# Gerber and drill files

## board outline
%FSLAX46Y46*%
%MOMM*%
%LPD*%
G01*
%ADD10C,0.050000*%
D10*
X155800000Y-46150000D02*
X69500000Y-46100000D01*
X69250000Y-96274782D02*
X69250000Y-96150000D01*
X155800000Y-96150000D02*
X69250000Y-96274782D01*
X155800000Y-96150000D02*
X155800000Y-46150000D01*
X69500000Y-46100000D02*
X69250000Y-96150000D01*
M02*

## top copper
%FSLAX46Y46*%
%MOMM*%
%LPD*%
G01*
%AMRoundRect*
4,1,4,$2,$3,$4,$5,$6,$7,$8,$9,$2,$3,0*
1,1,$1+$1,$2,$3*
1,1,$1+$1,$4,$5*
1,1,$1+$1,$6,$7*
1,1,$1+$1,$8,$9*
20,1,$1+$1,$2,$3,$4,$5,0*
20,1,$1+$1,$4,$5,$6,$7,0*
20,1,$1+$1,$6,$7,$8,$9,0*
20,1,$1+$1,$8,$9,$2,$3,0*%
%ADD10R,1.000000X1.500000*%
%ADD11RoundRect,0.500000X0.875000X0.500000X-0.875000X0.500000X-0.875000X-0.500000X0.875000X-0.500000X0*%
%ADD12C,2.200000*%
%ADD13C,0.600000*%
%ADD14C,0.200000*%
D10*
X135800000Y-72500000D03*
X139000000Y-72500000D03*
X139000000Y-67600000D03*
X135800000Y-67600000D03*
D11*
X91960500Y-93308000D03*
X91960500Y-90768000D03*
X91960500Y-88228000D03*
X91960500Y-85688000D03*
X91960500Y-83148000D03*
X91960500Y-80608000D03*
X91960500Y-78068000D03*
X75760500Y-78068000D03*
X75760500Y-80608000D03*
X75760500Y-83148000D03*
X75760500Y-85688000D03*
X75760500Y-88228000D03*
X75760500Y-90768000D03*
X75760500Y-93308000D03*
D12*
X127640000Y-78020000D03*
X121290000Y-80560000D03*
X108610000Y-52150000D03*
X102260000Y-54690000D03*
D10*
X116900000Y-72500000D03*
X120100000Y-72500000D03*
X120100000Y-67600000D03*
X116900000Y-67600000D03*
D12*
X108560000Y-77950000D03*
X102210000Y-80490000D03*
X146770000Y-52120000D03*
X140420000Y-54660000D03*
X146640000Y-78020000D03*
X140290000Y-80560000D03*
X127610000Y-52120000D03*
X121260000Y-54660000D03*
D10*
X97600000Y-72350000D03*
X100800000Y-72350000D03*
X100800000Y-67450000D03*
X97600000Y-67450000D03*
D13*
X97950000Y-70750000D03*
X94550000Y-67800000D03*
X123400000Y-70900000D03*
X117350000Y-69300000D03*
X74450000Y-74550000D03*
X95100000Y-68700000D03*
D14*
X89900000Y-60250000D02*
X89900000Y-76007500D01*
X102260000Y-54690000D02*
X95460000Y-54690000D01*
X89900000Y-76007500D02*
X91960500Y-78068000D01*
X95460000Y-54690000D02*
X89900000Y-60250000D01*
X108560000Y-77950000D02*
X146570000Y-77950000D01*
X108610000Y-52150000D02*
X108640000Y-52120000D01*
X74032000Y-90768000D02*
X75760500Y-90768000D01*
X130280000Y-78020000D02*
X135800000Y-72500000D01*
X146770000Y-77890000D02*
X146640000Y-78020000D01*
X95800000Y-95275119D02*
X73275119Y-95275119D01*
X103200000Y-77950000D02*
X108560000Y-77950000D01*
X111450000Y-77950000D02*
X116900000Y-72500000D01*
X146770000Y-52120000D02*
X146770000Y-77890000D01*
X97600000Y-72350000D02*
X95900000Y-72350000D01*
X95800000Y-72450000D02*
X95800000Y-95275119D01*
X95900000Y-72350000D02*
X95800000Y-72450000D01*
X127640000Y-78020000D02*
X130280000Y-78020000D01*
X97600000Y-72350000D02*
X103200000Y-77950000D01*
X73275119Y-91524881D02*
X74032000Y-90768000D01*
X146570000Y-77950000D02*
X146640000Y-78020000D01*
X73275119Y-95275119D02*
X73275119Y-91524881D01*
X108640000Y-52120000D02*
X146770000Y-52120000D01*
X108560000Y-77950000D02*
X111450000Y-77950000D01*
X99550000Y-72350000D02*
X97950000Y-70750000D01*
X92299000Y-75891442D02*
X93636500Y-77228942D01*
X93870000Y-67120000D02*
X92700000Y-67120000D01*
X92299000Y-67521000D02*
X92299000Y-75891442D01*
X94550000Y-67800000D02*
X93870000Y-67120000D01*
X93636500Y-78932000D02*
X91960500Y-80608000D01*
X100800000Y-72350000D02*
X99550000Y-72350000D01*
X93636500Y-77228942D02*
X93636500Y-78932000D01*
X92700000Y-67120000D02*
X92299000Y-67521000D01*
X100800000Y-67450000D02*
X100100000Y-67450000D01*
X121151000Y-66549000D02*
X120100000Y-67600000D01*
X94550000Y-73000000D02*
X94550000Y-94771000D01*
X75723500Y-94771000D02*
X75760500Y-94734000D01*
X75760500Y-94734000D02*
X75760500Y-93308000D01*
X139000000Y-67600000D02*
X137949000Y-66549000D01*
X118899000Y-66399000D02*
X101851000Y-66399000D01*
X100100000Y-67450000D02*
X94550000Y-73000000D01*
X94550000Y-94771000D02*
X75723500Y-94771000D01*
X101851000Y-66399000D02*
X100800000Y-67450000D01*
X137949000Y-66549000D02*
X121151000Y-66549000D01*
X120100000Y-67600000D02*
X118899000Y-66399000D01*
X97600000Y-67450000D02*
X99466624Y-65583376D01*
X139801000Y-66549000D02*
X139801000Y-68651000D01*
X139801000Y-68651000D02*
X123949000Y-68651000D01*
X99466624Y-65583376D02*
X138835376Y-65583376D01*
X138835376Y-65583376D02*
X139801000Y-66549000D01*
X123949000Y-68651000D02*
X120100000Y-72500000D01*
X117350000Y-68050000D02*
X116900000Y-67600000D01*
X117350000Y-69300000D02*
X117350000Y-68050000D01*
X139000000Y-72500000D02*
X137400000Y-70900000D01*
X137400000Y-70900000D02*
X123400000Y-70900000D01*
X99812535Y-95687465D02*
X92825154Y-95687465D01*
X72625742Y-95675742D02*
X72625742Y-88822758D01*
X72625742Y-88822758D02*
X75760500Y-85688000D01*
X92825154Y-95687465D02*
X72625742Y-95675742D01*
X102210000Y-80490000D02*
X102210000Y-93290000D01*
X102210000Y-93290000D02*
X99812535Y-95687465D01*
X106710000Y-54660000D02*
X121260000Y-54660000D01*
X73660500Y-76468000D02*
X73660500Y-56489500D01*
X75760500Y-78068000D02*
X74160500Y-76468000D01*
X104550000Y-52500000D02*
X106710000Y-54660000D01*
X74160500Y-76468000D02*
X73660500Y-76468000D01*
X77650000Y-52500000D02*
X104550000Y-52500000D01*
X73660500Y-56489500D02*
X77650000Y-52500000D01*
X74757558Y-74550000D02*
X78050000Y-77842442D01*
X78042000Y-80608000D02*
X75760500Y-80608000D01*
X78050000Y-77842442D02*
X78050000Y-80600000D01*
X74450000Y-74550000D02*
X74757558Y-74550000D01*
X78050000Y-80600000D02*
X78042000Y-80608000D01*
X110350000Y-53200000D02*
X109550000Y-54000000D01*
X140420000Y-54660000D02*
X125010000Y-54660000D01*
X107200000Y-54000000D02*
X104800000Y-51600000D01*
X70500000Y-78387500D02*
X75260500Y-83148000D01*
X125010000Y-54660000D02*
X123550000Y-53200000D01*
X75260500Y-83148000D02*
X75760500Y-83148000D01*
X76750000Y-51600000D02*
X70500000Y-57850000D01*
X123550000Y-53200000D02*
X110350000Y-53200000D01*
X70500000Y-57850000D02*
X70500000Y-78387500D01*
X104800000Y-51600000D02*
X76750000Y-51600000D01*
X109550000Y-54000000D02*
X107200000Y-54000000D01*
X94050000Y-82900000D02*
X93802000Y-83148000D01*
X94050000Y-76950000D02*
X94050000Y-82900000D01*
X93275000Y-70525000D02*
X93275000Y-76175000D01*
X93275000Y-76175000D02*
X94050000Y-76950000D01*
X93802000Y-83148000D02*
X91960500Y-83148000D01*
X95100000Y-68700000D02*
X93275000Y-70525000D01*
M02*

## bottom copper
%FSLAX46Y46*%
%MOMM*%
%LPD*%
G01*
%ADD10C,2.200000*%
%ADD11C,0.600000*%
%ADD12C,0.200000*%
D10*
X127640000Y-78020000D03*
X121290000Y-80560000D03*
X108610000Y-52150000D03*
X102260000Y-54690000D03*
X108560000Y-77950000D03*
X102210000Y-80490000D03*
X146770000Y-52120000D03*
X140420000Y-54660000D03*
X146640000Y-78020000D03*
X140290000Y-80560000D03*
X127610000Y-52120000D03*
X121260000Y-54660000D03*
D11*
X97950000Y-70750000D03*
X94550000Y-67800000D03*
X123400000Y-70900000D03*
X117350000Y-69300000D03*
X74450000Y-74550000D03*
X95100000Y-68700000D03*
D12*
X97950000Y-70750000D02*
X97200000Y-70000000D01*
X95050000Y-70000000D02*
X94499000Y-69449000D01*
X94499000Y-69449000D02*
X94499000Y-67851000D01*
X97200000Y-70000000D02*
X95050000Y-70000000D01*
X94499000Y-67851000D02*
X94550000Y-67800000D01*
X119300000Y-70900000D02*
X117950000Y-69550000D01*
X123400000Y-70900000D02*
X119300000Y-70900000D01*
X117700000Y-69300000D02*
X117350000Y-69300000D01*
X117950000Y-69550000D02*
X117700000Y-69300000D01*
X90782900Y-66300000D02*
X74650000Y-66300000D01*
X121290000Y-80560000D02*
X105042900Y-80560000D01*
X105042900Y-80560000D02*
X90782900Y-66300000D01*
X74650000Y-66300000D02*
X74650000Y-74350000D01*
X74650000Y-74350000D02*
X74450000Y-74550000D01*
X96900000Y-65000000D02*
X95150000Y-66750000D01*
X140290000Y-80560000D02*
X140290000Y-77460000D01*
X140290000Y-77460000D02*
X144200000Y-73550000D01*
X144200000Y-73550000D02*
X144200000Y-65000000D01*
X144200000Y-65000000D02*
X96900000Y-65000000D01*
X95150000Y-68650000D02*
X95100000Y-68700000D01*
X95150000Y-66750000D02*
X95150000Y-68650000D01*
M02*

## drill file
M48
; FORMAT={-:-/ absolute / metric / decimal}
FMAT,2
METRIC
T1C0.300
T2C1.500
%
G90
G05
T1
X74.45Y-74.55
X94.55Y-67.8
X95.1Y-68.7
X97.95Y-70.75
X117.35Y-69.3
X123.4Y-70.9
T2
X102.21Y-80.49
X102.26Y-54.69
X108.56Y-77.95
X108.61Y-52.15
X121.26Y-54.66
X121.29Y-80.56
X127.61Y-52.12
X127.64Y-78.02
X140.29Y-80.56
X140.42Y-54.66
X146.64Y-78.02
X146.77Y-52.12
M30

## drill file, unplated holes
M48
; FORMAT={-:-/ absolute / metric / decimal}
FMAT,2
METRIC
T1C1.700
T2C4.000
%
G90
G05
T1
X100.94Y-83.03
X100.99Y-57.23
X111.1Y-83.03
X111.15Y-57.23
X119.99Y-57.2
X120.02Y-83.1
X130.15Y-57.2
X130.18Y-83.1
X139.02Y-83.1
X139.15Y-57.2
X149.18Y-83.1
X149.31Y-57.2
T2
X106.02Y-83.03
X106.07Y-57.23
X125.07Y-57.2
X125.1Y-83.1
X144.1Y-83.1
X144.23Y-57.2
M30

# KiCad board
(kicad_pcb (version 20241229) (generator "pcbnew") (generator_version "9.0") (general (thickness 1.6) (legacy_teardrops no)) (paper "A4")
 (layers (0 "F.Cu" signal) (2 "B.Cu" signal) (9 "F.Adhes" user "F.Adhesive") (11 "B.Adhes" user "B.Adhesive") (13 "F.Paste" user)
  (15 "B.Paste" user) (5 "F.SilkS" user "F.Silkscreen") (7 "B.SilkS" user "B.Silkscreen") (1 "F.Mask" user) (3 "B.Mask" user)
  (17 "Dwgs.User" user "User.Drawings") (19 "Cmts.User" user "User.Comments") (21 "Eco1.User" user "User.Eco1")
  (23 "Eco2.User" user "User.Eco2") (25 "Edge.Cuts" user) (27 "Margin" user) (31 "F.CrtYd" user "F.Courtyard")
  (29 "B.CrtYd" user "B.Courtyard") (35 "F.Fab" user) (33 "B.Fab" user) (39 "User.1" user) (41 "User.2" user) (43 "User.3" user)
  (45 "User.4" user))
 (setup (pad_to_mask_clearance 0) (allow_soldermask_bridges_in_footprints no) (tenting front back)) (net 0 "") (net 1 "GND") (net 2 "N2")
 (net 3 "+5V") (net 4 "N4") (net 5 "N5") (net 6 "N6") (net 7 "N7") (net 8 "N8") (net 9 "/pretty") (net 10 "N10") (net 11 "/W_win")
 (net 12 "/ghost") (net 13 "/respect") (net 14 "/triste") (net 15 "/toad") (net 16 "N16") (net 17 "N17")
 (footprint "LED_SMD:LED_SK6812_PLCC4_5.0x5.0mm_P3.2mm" (layer "F.Cu") (at 137.4 70.05 90)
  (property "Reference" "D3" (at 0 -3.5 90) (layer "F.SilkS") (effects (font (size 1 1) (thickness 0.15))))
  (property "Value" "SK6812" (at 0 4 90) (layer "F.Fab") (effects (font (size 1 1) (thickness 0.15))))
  (pad "1" smd rect (at -2.45 -1.6 270) (size 1.5 1) (layers "F.Cu" "F.Mask" "F.Paste") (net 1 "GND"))
  (pad "2" smd rect (at -2.45 1.6 270) (size 1.5 1) (layers "F.Cu" "F.Mask" "F.Paste") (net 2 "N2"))
  (pad "3" smd rect (at 2.45 1.6 270) (size 1.5 1) (layers "F.Cu" "F.Mask" "F.Paste") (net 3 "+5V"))
  (pad "4" smd rect (at 2.45 -1.6 270) (size 1.5 1) (layers "F.Cu" "F.Mask" "F.Paste") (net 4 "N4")))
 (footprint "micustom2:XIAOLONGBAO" (layer "F.Cu") (at 83.8605 85.688 180)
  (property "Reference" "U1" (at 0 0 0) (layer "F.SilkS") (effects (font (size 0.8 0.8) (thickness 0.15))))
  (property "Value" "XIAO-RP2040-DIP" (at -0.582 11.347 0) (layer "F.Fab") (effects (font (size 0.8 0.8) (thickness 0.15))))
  (pad "1" smd roundrect (at -8.1 -7.62 180) (size 2.75 2) (layers "F.Cu" "F.Mask" "F.Paste") (roundrect_rratio 0.25) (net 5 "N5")
   (solder_mask_margin 0.102))
  (pad "2" smd roundrect (at -8.1 -5.08 180) (size 2.75 2) (layers "F.Cu" "F.Mask" "F.Paste") (roundrect_rratio 0.25) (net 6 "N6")
   (solder_mask_margin 0.102))
  (pad "3" smd roundrect (at -8.1 -2.54 180) (size 2.75 2) (layers "F.Cu" "F.Mask" "F.Paste") (roundrect_rratio 0.25) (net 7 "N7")
   (solder_mask_margin 0.102))
  (pad "4" smd roundrect (at -8.1 0 180) (size 2.75 2) (layers "F.Cu" "F.Mask" "F.Paste") (roundrect_rratio 0.25) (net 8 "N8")
   (solder_mask_margin 0.102))
  (pad "5" smd roundrect (at -8.1 2.54 180) (size 2.75 2) (layers "F.Cu" "F.Mask" "F.Paste") (roundrect_rratio 0.25) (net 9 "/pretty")
   (solder_mask_margin 0.102))
  (pad "6" smd roundrect (at -8.1 5.08 180) (size 2.75 2) (layers "F.Cu" "F.Mask" "F.Paste") (roundrect_rratio 0.25) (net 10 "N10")
   (solder_mask_margin 0.102))
  (pad "7" smd roundrect (at -8.1 7.62 180) (size 2.75 2) (layers "F.Cu" "F.Mask" "F.Paste") (roundrect_rratio 0.25) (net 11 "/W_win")
   (solder_mask_margin 0.102))
  (pad "8" smd roundrect (at 8.1 7.62 180) (size 2.75 2) (layers "F.Cu" "F.Mask" "F.Paste") (roundrect_rratio 0.25) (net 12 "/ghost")
   (solder_mask_margin 0.102))
  (pad "9" smd roundrect (at 8.1 5.08 180) (size 2.75 2) (layers "F.Cu" "F.Mask" "F.Paste") (roundrect_rratio 0.25) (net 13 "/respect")
   (solder_mask_margin 0.102))
  (pad "10" smd roundrect (at 8.1 2.54 180) (size 2.75 2) (layers "F.Cu" "F.Mask" "F.Paste") (roundrect_rratio 0.25) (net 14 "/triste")
   (solder_mask_margin 0.102))
  (pad "11" smd roundrect (at 8.1 0 180) (size 2.75 2) (layers "F.Cu" "F.Mask" "F.Paste") (roundrect_rratio 0.25) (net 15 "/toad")
   (solder_mask_margin 0.102))
  (pad "12" smd roundrect (at 8.1 -2.54 180) (size 2.75 2) (layers "F.Cu" "F.Mask" "F.Paste") (roundrect_rratio 0.25) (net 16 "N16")
   (solder_mask_margin 0.102))
  (pad "13" smd roundrect (at 8.1 -5.08 180) (size 2.75 2) (layers "F.Cu" "F.Mask" "F.Paste") (roundrect_rratio 0.25) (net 1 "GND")
   (solder_mask_margin 0.102))
  (pad "14" smd roundrect (at 8.1 -7.62 180) (size 2.75 2) (layers "F.Cu" "F.Mask" "F.Paste") (roundrect_rratio 0.25) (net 3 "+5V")
   (solder_mask_margin 0.102))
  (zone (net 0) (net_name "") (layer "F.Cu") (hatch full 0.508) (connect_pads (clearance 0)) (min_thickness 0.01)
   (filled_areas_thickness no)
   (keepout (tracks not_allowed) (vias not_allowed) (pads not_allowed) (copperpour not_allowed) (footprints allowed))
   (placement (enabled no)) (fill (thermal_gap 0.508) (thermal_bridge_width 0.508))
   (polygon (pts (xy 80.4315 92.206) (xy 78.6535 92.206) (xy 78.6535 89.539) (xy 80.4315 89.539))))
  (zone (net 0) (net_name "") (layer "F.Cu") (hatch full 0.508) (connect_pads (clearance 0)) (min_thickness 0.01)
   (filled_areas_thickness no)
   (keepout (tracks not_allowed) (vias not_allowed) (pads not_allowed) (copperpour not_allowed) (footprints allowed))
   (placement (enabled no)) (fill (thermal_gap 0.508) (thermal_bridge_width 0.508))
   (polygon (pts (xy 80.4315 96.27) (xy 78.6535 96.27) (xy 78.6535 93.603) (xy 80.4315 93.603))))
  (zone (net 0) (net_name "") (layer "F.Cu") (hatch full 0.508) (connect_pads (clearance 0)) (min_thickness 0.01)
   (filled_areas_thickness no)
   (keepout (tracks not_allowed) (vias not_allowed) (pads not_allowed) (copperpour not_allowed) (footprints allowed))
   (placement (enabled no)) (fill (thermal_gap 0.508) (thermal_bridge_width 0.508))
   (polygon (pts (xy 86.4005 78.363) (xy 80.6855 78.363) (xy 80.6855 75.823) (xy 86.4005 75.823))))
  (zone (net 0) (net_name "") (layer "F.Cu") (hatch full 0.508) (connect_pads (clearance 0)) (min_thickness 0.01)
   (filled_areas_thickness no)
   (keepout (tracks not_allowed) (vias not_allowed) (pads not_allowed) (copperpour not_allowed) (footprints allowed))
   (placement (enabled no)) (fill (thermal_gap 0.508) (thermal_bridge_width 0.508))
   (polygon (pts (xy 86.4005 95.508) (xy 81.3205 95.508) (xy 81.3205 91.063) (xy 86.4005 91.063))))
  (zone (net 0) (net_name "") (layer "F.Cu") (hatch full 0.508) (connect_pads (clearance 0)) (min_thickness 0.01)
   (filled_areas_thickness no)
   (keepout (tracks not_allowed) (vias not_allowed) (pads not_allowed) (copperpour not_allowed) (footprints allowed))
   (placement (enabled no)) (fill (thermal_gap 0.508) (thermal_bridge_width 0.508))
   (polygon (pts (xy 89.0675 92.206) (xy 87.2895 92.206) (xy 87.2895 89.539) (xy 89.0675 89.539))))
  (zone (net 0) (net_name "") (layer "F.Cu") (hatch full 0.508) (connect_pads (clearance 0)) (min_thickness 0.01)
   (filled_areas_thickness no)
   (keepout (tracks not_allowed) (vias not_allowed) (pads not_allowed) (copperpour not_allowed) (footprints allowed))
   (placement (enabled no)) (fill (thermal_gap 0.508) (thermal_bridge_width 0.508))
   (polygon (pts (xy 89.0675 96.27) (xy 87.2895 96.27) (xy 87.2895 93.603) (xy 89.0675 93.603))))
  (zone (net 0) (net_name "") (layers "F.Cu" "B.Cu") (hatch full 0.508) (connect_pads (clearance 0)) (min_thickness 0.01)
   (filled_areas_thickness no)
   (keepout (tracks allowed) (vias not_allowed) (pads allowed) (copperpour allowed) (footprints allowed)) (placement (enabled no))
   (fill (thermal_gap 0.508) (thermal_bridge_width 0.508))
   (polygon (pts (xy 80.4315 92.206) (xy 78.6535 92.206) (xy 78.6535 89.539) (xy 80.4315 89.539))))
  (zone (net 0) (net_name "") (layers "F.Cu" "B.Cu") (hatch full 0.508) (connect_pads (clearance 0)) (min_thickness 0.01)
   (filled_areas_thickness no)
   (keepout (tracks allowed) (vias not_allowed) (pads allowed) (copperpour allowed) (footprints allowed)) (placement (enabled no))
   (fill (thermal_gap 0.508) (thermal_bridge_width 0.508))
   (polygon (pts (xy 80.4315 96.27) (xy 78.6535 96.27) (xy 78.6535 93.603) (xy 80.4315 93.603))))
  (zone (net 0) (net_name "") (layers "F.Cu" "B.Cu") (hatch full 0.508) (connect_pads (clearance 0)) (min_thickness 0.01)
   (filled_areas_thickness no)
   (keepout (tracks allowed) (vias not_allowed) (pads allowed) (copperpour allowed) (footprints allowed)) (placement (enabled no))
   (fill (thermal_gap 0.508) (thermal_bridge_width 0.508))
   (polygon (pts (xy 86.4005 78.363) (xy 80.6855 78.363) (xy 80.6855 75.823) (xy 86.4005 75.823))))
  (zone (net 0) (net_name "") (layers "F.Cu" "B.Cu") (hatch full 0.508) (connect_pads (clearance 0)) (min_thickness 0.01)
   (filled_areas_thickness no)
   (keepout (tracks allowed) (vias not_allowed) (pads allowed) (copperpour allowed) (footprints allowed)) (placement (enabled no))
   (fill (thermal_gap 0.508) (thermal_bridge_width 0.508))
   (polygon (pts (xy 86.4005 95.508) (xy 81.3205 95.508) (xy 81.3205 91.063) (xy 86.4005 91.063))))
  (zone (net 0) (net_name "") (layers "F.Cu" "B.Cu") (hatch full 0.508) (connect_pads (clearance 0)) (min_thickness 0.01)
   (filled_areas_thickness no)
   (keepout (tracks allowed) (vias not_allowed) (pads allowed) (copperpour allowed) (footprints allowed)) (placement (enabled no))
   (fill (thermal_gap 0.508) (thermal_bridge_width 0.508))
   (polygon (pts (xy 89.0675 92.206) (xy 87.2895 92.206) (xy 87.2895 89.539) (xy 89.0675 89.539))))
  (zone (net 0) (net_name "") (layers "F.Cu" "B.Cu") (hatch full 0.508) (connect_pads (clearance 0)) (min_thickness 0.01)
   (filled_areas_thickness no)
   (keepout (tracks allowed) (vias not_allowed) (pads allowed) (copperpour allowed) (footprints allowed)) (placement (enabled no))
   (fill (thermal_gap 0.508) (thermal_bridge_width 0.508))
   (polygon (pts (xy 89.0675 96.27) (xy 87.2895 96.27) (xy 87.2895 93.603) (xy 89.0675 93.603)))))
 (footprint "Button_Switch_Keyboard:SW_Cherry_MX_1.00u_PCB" (layer "F.Cu") (at 127.64 78.02)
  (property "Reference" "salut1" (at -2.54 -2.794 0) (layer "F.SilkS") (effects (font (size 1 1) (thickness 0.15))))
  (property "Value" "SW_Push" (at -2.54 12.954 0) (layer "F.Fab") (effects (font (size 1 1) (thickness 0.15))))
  (pad "" np_thru_hole circle (at -7.62 5.08) (size 1.7 1.7) (drill 1.7) (layers "*.Cu" "*.Mask"))
  (pad "" np_thru_hole circle (at -2.54 5.08) (size 4 4) (drill 4) (layers "*.Cu" "*.Mask"))
  (pad "" np_thru_hole circle (at 2.54 5.08) (size 1.7 1.7) (drill 1.7) (layers "*.Cu" "*.Mask"))
  (pad "1" thru_hole circle (at 0 0) (size 2.2 2.2) (drill 1.5) (layers "*.Cu" "*.Mask") (remove_unused_layers no) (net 1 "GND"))
  (pad "2" thru_hole circle (at -6.35 2.54) (size 2.2 2.2) (drill 1.5) (layers "*.Cu" "*.Mask") (remove_unused_layers no)
   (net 13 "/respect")))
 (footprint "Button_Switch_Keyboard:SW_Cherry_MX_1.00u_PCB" (layer "F.Cu") (at 108.61 52.15)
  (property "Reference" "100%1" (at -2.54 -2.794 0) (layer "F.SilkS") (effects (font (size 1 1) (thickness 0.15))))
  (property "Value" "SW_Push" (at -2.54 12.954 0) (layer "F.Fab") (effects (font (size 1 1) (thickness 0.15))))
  (pad "" np_thru_hole circle (at -7.62 5.08) (size 1.7 1.7) (drill 1.7) (layers "*.Cu" "*.Mask"))
  (pad "" np_thru_hole circle (at -2.54 5.08) (size 4 4) (drill 4) (layers "*.Cu" "*.Mask"))
  (pad "" np_thru_hole circle (at 2.54 5.08) (size 1.7 1.7) (drill 1.7) (layers "*.Cu" "*.Mask"))
  (pad "1" thru_hole circle (at 0 0) (size 2.2 2.2) (drill 1.5) (layers "*.Cu" "*.Mask") (remove_unused_layers no) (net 1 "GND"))
  (pad "2" thru_hole circle (at -6.35 2.54) (size 2.2 2.2) (drill 1.5) (layers "*.Cu" "*.Mask") (remove_unused_layers no) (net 11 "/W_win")))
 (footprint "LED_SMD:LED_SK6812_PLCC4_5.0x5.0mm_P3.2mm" (layer "F.Cu") (at 118.5 70.05 90)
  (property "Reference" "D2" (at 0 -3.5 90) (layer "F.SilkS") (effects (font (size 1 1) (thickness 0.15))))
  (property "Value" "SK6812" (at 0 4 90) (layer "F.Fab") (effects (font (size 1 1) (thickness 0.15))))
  (pad "1" smd rect (at -2.45 -1.6 270) (size 1.5 1) (layers "F.Cu" "F.Mask" "F.Paste") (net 1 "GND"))
  (pad "2" smd rect (at -2.45 1.6 270) (size 1.5 1) (layers "F.Cu" "F.Mask" "F.Paste") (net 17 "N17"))
  (pad "3" smd rect (at 2.45 1.6 270) (size 1.5 1) (layers "F.Cu" "F.Mask" "F.Paste") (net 3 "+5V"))
  (pad "4" smd rect (at 2.45 -1.6 270) (size 1.5 1) (layers "F.Cu" "F.Mask" "F.Paste") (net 2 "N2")))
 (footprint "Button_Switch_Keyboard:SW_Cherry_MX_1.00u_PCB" (layer "F.Cu") (at 108.56 77.95)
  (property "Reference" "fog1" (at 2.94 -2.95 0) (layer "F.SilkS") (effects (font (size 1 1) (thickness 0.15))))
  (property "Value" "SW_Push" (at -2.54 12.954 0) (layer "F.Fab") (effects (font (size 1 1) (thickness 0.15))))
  (pad "" np_thru_hole circle (at -7.62 5.08) (size 1.7 1.7) (drill 1.7) (layers "*.Cu" "*.Mask"))
  (pad "" np_thru_hole circle (at -2.54 5.08) (size 4 4) (drill 4) (layers "*.Cu" "*.Mask"))
  (pad "" np_thru_hole circle (at 2.54 5.08) (size 1.7 1.7) (drill 1.7) (layers "*.Cu" "*.Mask"))
  (pad "1" thru_hole circle (at 0 0) (size 2.2 2.2) (drill 1.5) (layers "*.Cu" "*.Mask") (remove_unused_layers no) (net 1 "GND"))
  (pad "2" thru_hole circle (at -6.35 2.54) (size 2.2 2.2) (drill 1.5) (layers "*.Cu" "*.Mask") (remove_unused_layers no) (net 15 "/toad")))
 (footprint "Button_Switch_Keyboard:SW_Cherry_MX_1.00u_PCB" (layer "F.Cu") (at 146.77 52.12)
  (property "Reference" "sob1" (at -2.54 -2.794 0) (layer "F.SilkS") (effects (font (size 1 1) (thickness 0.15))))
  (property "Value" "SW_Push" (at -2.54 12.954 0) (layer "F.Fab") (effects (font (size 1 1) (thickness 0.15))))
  (pad "" np_thru_hole circle (at -7.62 5.08) (size 1.7 1.7) (drill 1.7) (layers "*.Cu" "*.Mask"))
  (pad "" np_thru_hole circle (at -2.54 5.08) (size 4 4) (drill 4) (layers "*.Cu" "*.Mask"))
  (pad "" np_thru_hole circle (at 2.54 5.08) (size 1.7 1.7) (drill 1.7) (layers "*.Cu" "*.Mask"))
  (pad "1" thru_hole circle (at 0 0) (size 2.2 2.2) (drill 1.5) (layers "*.Cu" "*.Mask") (remove_unused_layers no) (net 1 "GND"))
  (pad "2" thru_hole circle (at -6.35 2.54) (size 2.2 2.2) (drill 1.5) (layers "*.Cu" "*.Mask") (remove_unused_layers no) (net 14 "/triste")))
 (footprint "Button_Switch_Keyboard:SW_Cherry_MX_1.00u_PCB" (layer "F.Cu") (at 146.64 78.02)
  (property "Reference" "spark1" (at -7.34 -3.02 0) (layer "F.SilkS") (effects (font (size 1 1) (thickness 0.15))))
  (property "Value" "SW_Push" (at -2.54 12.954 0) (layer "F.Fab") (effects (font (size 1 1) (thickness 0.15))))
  (pad "" np_thru_hole circle (at -7.62 5.08) (size 1.7 1.7) (drill 1.7) (layers "*.Cu" "*.Mask"))
  (pad "" np_thru_hole circle (at -2.54 5.08) (size 4 4) (drill 4) (layers "*.Cu" "*.Mask"))
  (pad "" np_thru_hole circle (at 2.54 5.08) (size 1.7 1.7) (drill 1.7) (layers "*.Cu" "*.Mask"))
  (pad "1" thru_hole circle (at 0 0) (size 2.2 2.2) (drill 1.5) (layers "*.Cu" "*.Mask") (remove_unused_layers no) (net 1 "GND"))
  (pad "2" thru_hole circle (at -6.35 2.54) (size 2.2 2.2) (drill 1.5) (layers "*.Cu" "*.Mask") (remove_unused_layers no) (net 9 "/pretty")))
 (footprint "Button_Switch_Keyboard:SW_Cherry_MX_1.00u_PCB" (layer "F.Cu") (at 127.61 52.12)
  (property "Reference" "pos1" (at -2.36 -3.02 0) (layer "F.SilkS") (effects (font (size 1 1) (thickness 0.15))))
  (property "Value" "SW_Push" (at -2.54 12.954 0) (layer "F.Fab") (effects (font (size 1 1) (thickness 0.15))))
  (pad "" np_thru_hole circle (at -7.62 5.08) (size 1.7 1.7) (drill 1.7) (layers "*.Cu" "*.Mask"))
  (pad "" np_thru_hole circle (at -2.54 5.08) (size 4 4) (drill 4) (layers "*.Cu" "*.Mask"))
  (pad "" np_thru_hole circle (at 2.54 5.08) (size 1.7 1.7) (drill 1.7) (layers "*.Cu" "*.Mask"))
  (pad "1" thru_hole circle (at 0 0) (size 2.2 2.2) (drill 1.5) (layers "*.Cu" "*.Mask") (remove_unused_layers no) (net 1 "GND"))
  (pad "2" thru_hole circle (at -6.35 2.54) (size 2.2 2.2) (drill 1.5) (layers "*.Cu" "*.Mask") (remove_unused_layers no) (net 12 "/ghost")))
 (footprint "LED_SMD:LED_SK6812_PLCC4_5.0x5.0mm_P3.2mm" (layer "F.Cu") (at 99.2 69.9 90)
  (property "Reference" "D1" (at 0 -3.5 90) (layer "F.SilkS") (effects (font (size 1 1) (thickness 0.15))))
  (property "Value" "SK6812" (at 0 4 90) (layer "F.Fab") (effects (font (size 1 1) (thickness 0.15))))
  (pad "1" smd rect (at -2.45 -1.6 270) (size 1.5 1) (layers "F.Cu" "F.Mask" "F.Paste") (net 1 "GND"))
  (pad "2" smd rect (at -2.45 1.6 270) (size 1.5 1) (layers "F.Cu" "F.Mask" "F.Paste") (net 10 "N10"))
  (pad "3" smd rect (at 2.45 1.6 270) (size 1.5 1) (layers "F.Cu" "F.Mask" "F.Paste") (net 3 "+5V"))
  (pad "4" smd rect (at 2.45 -1.6 270) (size 1.5 1) (layers "F.Cu" "F.Mask" "F.Paste") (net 17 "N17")))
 (gr_line (start 155.8 46.15) (end 69.5 46.1) (stroke (width 0.05) (type default)) (layer "Edge.Cuts"))
 (gr_line (start 69.25 96.274782) (end 69.25 96.15) (stroke (width 0.05) (type default)) (layer "Edge.Cuts"))
 (gr_line (start 155.8 96.15) (end 69.25 96.274782) (stroke (width 0.05) (type default)) (layer "Edge.Cuts"))
 (gr_line (start 155.8 96.15) (end 155.8 46.15) (stroke (width 0.05) (type default)) (layer "Edge.Cuts"))
 (gr_line (start 69.5 46.1) (end 69.25 96.15) (stroke (width 0.05) (type default)) (layer "Edge.Cuts"))
 (segment (start 89.9 60.25) (end 89.9 76.0075) (width 0.2) (layer "F.Cu") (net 11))
 (segment (start 102.26 54.69) (end 95.46 54.69) (width 0.2) (layer "F.Cu") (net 11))
 (segment (start 89.9 76.0075) (end 91.9605 78.068) (width 0.2) (layer "F.Cu") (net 11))
 (segment (start 95.46 54.69) (end 89.9 60.25) (width 0.2) (layer "F.Cu") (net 11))
 (segment (start 89.9 60.25) (end 89.8605 60.2895) (width 0.2) (layer "F.Cu") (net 11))
 (segment (start 108.56 77.95) (end 146.57 77.95) (width 0.2) (layer "F.Cu") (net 1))
 (segment (start 108.61 52.15) (end 108.64 52.12) (width 0.2) (layer "F.Cu") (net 1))
 (segment (start 74.032 90.768) (end 75.7605 90.768) (width 0.2) (layer "F.Cu") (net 1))
 (segment (start 130.28 78.02) (end 135.8 72.5) (width 0.2) (layer "F.Cu") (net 1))
 (segment (start 146.77 77.89) (end 146.64 78.02) (width 0.2) (layer "F.Cu") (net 1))
 (segment (start 95.8 95.275119) (end 73.275119 95.275119) (width 0.2) (layer "F.Cu") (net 1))
 (segment (start 103.2 77.95) (end 108.56 77.95) (width 0.2) (layer "F.Cu") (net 1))
 (segment (start 111.45 77.95) (end 116.9 72.5) (width 0.2) (layer "F.Cu") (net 1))
 (segment (start 146.77 52.12) (end 146.77 77.89) (width 0.2) (layer "F.Cu") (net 1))
 (segment (start 97.6 72.35) (end 95.9 72.35) (width 0.2) (layer "F.Cu") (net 1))
 (segment (start 95.8 72.45) (end 95.8 95.275119) (width 0.2) (layer "F.Cu") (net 1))
 (segment (start 95.9 72.35) (end 95.8 72.45) (width 0.2) (layer "F.Cu") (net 1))
 (segment (start 127.64 78.02) (end 130.28 78.02) (width 0.2) (layer "F.Cu") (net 1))
 (segment (start 97.6 72.35) (end 103.2 77.95) (width 0.2) (layer "F.Cu") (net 1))
 (segment (start 73.275119 91.524881) (end 74.032 90.768) (width 0.2) (layer "F.Cu") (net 1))
 (segment (start 146.57 77.95) (end 146.64 78.02) (width 0.2) (layer "F.Cu") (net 1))
 (segment (start 73.275119 95.275119) (end 73.275119 91.524881) (width 0.2) (layer "F.Cu") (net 1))
 (segment (start 108.64 52.12) (end 146.77 52.12) (width 0.2) (layer "F.Cu") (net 1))
 (segment (start 108.56 77.95) (end 111.45 77.95) (width 0.2) (layer "F.Cu") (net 1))
 (segment (start 99.55 72.35) (end 97.95 70.75) (width 0.2) (layer "F.Cu") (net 10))
 (segment (start 92.299 75.891442) (end 93.6365 77.228942) (width 0.2) (layer "F.Cu") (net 10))
 (segment (start 93.87 67.12) (end 92.7 67.12) (width 0.2) (layer "F.Cu") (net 10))
 (segment (start 92.299 67.521) (end 92.299 75.891442) (width 0.2) (layer "F.Cu") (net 10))
 (segment (start 94.55 67.8) (end 93.87 67.12) (width 0.2) (layer "F.Cu") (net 10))
 (segment (start 93.6365 78.932) (end 91.9605 80.608) (width 0.2) (layer "F.Cu") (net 10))
 (segment (start 100.8 72.35) (end 99.55 72.35) (width 0.2) (layer "F.Cu") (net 10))
 (segment (start 93.6365 77.228942) (end 93.6365 78.932) (width 0.2) (layer "F.Cu") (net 10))
 (segment (start 92.7 67.12) (end 92.299 67.521) (width 0.2) (layer "F.Cu") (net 10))
 (via (at 97.95 70.75) (size 0.6) (drill 0.3) (layers "F.Cu" "B.Cu") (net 10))
 (via (at 94.55 67.8) (size 0.6) (drill 0.3) (layers "F.Cu" "B.Cu") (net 10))
 (segment (start 97.95 70.75) (end 97.2 70) (width 0.2) (layer "B.Cu") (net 10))
 (segment (start 95.05 70) (end 94.499 69.449) (width 0.2) (layer "B.Cu") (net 10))
 (segment (start 94.499 69.449) (end 94.499 67.851) (width 0.2) (layer "B.Cu") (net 10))
 (segment (start 97.2 70) (end 95.05 70) (width 0.2) (layer "B.Cu") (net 10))
 (segment (start 94.499 67.851) (end 94.55 67.8) (width 0.2) (layer "B.Cu") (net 10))
 (segment (start 100.8 67.45) (end 100.1 67.45) (width 0.2) (layer "F.Cu") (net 3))
 (segment (start 121.151 66.549) (end 120.1 67.6) (width 0.2) (layer "F.Cu") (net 3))
 (segment (start 94.55 73) (end 94.55 94.771) (width 0.2) (layer "F.Cu") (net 3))
 (segment (start 75.7235 94.771) (end 75.7605 94.734) (width 0.2) (layer "F.Cu") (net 3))
 (segment (start 75.7605 94.734) (end 75.7605 93.308) (width 0.2) (layer "F.Cu") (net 3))
 (segment (start 139 67.6) (end 137.949 66.549) (width 0.2) (layer "F.Cu") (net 3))
 (segment (start 118.899 66.399) (end 101.851 66.399) (width 0.2) (layer "F.Cu") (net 3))
 (segment (start 100.1 67.45) (end 94.55 73) (width 0.2) (layer "F.Cu") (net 3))
 (segment (start 94.55 94.771) (end 75.7235 94.771) (width 0.2) (layer "F.Cu") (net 3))
 (segment (start 101.851 66.399) (end 100.8 67.45) (width 0.2) (layer "F.Cu") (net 3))
 (segment (start 137.949 66.549) (end 121.151 66.549) (width 0.2) (layer "F.Cu") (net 3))
 (segment (start 120.1 67.6) (end 118.899 66.399) (width 0.2) (layer "F.Cu") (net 3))
 (segment (start 97.6 67.45) (end 99.466624 65.583376) (width 0.2) (layer "F.Cu") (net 17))
 (segment (start 139.801 66.549) (end 139.801 68.651) (width 0.2) (layer "F.Cu") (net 17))
 (segment (start 139.801 68.651) (end 123.949 68.651) (width 0.2) (layer "F.Cu") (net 17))
 (segment (start 99.466624 65.583376) (end 138.835376 65.583376) (width 0.2) (layer "F.Cu") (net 17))
 (segment (start 138.835376 65.583376) (end 139.801 66.549) (width 0.2) (layer "F.Cu") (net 17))
 (segment (start 123.949 68.651) (end 120.1 72.5) (width 0.2) (layer "F.Cu") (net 17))
 (segment (start 117.35 68.05) (end 116.9 67.6) (width 0.2) (layer "F.Cu") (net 2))
 (segment (start 117.35 69.3) (end 117.35 68.05) (width 0.2) (layer "F.Cu") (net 2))
 (segment (start 139 72.5) (end 137.4 70.9) (width 0.2) (layer "F.Cu") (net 2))
 (segment (start 137.4 70.9) (end 123.4 70.9) (width 0.2) (layer "F.Cu") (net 2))
 (via (at 123.4 70.9) (size 0.6) (drill 0.3) (layers "F.Cu" "B.Cu") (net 2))
 (via (at 117.35 69.3) (size 0.6) (drill 0.3) (layers "F.Cu" "B.Cu") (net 2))
 (segment (start 119.3 70.9) (end 117.95 69.55) (width 0.2) (layer "B.Cu") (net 2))
 (segment (start 123.4 70.9) (end 119.3 70.9) (width 0.2) (layer "B.Cu") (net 2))
 (segment (start 117.7 69.3) (end 117.35 69.3) (width 0.2) (layer "B.Cu") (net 2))
 (segment (start 117.95 69.55) (end 117.7 69.3) (width 0.2) (layer "B.Cu") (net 2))
 (segment (start 99.812535 95.687465) (end 92.825154 95.687465) (width 0.2) (layer "F.Cu") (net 15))
 (segment (start 72.625742 95.675742) (end 72.625742 88.822758) (width 0.2) (layer "F.Cu") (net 15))
 (segment (start 72.625742 88.822758) (end 75.7605 85.688) (width 0.2) (layer "F.Cu") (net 15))
 (segment (start 92.825154 95.687465) (end 72.625742 95.675742) (width 0.2) (layer "F.Cu") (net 15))
 (segment (start 102.21 80.49) (end 102.21 93.29) (width 0.2) (layer "F.Cu") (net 15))
 (segment (start 102.21 93.29) (end 99.812535 95.687465) (width 0.2) (layer "F.Cu") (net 15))
 (segment (start 106.71 54.66) (end 121.26 54.66) (width 0.2) (layer "F.Cu") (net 12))
 (segment (start 73.6605 76.468) (end 73.6605 56.4895) (width 0.2) (layer "F.Cu") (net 12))
 (segment (start 104.55 52.5) (end 106.71 54.66) (width 0.2) (layer "F.Cu") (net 12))
 (segment (start 77.65 52.5) (end 104.55 52.5) (width 0.2) (layer "F.Cu") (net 12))
 (segment (start 73.6605 56.4895) (end 77.65 52.5) (width 0.2) (layer "F.Cu") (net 12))
 (segment (start 74.757558 74.55) (end 78.05 77.842442) (width 0.2) (layer "F.Cu") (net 13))
 (segment (start 78.042 80.608) (end 75.7605 80.608) (width 0.2) (layer "F.Cu") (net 13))
 (segment (start 78.05 77.842442) (end 78.05 80.6) (width 0.2) (layer "F.Cu") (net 13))
 (segment (start 74.45 74.55) (end 74.757558 74.55) (width 0.2) (layer "F.Cu") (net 13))
 (segment (start 78.05 80.6) (end 78.042 80.608) (width 0.2) (layer "F.Cu") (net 13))
 (via (at 74.45 74.55) (size 0.6) (drill 0.3) (layers "F.Cu" "B.Cu") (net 13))
 (segment (start 90.7829 66.3) (end 74.65 66.3) (width 0.2) (layer "B.Cu") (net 13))
 (segment (start 121.29 80.56) (end 105.0429 80.56) (width 0.2) (layer "B.Cu") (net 13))
 (segment (start 105.0429 80.56) (end 90.7829 66.3) (width 0.2) (layer "B.Cu") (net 13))
 (segment (start 74.65 66.3) (end 74.65 74.35) (width 0.2) (layer "B.Cu") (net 13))
 (segment (start 74.65 74.35) (end 74.45 74.55) (width 0.2) (layer "B.Cu") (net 13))
 (segment (start 110.35 53.2) (end 109.55 54) (width 0.2) (layer "F.Cu") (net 14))
 (segment (start 140.42 54.66) (end 125.01 54.66) (width 0.2) (layer "F.Cu") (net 14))
 (segment (start 107.2 54) (end 104.8 51.6) (width 0.2) (layer "F.Cu") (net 14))
 (segment (start 70.5 78.3875) (end 75.2605 83.148) (width 0.2) (layer "F.Cu") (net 14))
 (segment (start 125.01 54.66) (end 123.55 53.2) (width 0.2) (layer "F.Cu") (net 14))
 (segment (start 75.2605 83.148) (end 75.7605 83.148) (width 0.2) (layer "F.Cu") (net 14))
 (segment (start 76.75 51.6) (end 70.5 57.85) (width 0.2) (layer "F.Cu") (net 14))
 (segment (start 123.55 53.2) (end 110.35 53.2) (width 0.2) (layer "F.Cu") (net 14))
 (segment (start 70.5 57.85) (end 70.5 78.3875) (width 0.2) (layer "F.Cu") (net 14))
 (segment (start 104.8 51.6) (end 76.75 51.6) (width 0.2) (layer "F.Cu") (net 14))
 (segment (start 109.55 54) (end 107.2 54) (width 0.2) (layer "F.Cu") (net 14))
 (segment (start 94.05 82.9) (end 93.802 83.148) (width 0.2) (layer "F.Cu") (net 9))
 (segment (start 94.05 76.95) (end 94.05 82.9) (width 0.2) (layer "F.Cu") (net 9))
 (segment (start 93.275 70.525) (end 93.275 76.175) (width 0.2) (layer "F.Cu") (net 9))
 (segment (start 93.275 76.175) (end 94.05 76.95) (width 0.2) (layer "F.Cu") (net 9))
 (segment (start 93.802 83.148) (end 91.9605 83.148) (width 0.2) (layer "F.Cu") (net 9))
 (segment (start 95.1 68.7) (end 93.275 70.525) (width 0.2) (layer "F.Cu") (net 9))
 (segment (start 93.275 70.525) (end 93.25 70.55) (width 0.2) (layer "F.Cu") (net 9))
 (via (at 95.1 68.7) (size 0.6) (drill 0.3) (layers "F.Cu" "B.Cu") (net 9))
 (segment (start 96.9 65) (end 95.15 66.75) (width 0.2) (layer "B.Cu") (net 9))
 (segment (start 140.29 80.56) (end 140.29 77.46) (width 0.2) (layer "B.Cu") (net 9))
 (segment (start 140.29 77.46) (end 144.2 73.55) (width 0.2) (layer "B.Cu") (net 9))
 (segment (start 144.2 73.55) (end 144.2 65) (width 0.2) (layer "B.Cu") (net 9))
 (segment (start 144.2 65) (end 96.9 65) (width 0.2) (layer "B.Cu") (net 9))
 (segment (start 95.15 68.65) (end 95.1 68.7) (width 0.2) (layer "B.Cu") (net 9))
 (segment (start 95.15 66.75) (end 95.15 68.65) (width 0.2) (layer "B.Cu") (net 9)))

